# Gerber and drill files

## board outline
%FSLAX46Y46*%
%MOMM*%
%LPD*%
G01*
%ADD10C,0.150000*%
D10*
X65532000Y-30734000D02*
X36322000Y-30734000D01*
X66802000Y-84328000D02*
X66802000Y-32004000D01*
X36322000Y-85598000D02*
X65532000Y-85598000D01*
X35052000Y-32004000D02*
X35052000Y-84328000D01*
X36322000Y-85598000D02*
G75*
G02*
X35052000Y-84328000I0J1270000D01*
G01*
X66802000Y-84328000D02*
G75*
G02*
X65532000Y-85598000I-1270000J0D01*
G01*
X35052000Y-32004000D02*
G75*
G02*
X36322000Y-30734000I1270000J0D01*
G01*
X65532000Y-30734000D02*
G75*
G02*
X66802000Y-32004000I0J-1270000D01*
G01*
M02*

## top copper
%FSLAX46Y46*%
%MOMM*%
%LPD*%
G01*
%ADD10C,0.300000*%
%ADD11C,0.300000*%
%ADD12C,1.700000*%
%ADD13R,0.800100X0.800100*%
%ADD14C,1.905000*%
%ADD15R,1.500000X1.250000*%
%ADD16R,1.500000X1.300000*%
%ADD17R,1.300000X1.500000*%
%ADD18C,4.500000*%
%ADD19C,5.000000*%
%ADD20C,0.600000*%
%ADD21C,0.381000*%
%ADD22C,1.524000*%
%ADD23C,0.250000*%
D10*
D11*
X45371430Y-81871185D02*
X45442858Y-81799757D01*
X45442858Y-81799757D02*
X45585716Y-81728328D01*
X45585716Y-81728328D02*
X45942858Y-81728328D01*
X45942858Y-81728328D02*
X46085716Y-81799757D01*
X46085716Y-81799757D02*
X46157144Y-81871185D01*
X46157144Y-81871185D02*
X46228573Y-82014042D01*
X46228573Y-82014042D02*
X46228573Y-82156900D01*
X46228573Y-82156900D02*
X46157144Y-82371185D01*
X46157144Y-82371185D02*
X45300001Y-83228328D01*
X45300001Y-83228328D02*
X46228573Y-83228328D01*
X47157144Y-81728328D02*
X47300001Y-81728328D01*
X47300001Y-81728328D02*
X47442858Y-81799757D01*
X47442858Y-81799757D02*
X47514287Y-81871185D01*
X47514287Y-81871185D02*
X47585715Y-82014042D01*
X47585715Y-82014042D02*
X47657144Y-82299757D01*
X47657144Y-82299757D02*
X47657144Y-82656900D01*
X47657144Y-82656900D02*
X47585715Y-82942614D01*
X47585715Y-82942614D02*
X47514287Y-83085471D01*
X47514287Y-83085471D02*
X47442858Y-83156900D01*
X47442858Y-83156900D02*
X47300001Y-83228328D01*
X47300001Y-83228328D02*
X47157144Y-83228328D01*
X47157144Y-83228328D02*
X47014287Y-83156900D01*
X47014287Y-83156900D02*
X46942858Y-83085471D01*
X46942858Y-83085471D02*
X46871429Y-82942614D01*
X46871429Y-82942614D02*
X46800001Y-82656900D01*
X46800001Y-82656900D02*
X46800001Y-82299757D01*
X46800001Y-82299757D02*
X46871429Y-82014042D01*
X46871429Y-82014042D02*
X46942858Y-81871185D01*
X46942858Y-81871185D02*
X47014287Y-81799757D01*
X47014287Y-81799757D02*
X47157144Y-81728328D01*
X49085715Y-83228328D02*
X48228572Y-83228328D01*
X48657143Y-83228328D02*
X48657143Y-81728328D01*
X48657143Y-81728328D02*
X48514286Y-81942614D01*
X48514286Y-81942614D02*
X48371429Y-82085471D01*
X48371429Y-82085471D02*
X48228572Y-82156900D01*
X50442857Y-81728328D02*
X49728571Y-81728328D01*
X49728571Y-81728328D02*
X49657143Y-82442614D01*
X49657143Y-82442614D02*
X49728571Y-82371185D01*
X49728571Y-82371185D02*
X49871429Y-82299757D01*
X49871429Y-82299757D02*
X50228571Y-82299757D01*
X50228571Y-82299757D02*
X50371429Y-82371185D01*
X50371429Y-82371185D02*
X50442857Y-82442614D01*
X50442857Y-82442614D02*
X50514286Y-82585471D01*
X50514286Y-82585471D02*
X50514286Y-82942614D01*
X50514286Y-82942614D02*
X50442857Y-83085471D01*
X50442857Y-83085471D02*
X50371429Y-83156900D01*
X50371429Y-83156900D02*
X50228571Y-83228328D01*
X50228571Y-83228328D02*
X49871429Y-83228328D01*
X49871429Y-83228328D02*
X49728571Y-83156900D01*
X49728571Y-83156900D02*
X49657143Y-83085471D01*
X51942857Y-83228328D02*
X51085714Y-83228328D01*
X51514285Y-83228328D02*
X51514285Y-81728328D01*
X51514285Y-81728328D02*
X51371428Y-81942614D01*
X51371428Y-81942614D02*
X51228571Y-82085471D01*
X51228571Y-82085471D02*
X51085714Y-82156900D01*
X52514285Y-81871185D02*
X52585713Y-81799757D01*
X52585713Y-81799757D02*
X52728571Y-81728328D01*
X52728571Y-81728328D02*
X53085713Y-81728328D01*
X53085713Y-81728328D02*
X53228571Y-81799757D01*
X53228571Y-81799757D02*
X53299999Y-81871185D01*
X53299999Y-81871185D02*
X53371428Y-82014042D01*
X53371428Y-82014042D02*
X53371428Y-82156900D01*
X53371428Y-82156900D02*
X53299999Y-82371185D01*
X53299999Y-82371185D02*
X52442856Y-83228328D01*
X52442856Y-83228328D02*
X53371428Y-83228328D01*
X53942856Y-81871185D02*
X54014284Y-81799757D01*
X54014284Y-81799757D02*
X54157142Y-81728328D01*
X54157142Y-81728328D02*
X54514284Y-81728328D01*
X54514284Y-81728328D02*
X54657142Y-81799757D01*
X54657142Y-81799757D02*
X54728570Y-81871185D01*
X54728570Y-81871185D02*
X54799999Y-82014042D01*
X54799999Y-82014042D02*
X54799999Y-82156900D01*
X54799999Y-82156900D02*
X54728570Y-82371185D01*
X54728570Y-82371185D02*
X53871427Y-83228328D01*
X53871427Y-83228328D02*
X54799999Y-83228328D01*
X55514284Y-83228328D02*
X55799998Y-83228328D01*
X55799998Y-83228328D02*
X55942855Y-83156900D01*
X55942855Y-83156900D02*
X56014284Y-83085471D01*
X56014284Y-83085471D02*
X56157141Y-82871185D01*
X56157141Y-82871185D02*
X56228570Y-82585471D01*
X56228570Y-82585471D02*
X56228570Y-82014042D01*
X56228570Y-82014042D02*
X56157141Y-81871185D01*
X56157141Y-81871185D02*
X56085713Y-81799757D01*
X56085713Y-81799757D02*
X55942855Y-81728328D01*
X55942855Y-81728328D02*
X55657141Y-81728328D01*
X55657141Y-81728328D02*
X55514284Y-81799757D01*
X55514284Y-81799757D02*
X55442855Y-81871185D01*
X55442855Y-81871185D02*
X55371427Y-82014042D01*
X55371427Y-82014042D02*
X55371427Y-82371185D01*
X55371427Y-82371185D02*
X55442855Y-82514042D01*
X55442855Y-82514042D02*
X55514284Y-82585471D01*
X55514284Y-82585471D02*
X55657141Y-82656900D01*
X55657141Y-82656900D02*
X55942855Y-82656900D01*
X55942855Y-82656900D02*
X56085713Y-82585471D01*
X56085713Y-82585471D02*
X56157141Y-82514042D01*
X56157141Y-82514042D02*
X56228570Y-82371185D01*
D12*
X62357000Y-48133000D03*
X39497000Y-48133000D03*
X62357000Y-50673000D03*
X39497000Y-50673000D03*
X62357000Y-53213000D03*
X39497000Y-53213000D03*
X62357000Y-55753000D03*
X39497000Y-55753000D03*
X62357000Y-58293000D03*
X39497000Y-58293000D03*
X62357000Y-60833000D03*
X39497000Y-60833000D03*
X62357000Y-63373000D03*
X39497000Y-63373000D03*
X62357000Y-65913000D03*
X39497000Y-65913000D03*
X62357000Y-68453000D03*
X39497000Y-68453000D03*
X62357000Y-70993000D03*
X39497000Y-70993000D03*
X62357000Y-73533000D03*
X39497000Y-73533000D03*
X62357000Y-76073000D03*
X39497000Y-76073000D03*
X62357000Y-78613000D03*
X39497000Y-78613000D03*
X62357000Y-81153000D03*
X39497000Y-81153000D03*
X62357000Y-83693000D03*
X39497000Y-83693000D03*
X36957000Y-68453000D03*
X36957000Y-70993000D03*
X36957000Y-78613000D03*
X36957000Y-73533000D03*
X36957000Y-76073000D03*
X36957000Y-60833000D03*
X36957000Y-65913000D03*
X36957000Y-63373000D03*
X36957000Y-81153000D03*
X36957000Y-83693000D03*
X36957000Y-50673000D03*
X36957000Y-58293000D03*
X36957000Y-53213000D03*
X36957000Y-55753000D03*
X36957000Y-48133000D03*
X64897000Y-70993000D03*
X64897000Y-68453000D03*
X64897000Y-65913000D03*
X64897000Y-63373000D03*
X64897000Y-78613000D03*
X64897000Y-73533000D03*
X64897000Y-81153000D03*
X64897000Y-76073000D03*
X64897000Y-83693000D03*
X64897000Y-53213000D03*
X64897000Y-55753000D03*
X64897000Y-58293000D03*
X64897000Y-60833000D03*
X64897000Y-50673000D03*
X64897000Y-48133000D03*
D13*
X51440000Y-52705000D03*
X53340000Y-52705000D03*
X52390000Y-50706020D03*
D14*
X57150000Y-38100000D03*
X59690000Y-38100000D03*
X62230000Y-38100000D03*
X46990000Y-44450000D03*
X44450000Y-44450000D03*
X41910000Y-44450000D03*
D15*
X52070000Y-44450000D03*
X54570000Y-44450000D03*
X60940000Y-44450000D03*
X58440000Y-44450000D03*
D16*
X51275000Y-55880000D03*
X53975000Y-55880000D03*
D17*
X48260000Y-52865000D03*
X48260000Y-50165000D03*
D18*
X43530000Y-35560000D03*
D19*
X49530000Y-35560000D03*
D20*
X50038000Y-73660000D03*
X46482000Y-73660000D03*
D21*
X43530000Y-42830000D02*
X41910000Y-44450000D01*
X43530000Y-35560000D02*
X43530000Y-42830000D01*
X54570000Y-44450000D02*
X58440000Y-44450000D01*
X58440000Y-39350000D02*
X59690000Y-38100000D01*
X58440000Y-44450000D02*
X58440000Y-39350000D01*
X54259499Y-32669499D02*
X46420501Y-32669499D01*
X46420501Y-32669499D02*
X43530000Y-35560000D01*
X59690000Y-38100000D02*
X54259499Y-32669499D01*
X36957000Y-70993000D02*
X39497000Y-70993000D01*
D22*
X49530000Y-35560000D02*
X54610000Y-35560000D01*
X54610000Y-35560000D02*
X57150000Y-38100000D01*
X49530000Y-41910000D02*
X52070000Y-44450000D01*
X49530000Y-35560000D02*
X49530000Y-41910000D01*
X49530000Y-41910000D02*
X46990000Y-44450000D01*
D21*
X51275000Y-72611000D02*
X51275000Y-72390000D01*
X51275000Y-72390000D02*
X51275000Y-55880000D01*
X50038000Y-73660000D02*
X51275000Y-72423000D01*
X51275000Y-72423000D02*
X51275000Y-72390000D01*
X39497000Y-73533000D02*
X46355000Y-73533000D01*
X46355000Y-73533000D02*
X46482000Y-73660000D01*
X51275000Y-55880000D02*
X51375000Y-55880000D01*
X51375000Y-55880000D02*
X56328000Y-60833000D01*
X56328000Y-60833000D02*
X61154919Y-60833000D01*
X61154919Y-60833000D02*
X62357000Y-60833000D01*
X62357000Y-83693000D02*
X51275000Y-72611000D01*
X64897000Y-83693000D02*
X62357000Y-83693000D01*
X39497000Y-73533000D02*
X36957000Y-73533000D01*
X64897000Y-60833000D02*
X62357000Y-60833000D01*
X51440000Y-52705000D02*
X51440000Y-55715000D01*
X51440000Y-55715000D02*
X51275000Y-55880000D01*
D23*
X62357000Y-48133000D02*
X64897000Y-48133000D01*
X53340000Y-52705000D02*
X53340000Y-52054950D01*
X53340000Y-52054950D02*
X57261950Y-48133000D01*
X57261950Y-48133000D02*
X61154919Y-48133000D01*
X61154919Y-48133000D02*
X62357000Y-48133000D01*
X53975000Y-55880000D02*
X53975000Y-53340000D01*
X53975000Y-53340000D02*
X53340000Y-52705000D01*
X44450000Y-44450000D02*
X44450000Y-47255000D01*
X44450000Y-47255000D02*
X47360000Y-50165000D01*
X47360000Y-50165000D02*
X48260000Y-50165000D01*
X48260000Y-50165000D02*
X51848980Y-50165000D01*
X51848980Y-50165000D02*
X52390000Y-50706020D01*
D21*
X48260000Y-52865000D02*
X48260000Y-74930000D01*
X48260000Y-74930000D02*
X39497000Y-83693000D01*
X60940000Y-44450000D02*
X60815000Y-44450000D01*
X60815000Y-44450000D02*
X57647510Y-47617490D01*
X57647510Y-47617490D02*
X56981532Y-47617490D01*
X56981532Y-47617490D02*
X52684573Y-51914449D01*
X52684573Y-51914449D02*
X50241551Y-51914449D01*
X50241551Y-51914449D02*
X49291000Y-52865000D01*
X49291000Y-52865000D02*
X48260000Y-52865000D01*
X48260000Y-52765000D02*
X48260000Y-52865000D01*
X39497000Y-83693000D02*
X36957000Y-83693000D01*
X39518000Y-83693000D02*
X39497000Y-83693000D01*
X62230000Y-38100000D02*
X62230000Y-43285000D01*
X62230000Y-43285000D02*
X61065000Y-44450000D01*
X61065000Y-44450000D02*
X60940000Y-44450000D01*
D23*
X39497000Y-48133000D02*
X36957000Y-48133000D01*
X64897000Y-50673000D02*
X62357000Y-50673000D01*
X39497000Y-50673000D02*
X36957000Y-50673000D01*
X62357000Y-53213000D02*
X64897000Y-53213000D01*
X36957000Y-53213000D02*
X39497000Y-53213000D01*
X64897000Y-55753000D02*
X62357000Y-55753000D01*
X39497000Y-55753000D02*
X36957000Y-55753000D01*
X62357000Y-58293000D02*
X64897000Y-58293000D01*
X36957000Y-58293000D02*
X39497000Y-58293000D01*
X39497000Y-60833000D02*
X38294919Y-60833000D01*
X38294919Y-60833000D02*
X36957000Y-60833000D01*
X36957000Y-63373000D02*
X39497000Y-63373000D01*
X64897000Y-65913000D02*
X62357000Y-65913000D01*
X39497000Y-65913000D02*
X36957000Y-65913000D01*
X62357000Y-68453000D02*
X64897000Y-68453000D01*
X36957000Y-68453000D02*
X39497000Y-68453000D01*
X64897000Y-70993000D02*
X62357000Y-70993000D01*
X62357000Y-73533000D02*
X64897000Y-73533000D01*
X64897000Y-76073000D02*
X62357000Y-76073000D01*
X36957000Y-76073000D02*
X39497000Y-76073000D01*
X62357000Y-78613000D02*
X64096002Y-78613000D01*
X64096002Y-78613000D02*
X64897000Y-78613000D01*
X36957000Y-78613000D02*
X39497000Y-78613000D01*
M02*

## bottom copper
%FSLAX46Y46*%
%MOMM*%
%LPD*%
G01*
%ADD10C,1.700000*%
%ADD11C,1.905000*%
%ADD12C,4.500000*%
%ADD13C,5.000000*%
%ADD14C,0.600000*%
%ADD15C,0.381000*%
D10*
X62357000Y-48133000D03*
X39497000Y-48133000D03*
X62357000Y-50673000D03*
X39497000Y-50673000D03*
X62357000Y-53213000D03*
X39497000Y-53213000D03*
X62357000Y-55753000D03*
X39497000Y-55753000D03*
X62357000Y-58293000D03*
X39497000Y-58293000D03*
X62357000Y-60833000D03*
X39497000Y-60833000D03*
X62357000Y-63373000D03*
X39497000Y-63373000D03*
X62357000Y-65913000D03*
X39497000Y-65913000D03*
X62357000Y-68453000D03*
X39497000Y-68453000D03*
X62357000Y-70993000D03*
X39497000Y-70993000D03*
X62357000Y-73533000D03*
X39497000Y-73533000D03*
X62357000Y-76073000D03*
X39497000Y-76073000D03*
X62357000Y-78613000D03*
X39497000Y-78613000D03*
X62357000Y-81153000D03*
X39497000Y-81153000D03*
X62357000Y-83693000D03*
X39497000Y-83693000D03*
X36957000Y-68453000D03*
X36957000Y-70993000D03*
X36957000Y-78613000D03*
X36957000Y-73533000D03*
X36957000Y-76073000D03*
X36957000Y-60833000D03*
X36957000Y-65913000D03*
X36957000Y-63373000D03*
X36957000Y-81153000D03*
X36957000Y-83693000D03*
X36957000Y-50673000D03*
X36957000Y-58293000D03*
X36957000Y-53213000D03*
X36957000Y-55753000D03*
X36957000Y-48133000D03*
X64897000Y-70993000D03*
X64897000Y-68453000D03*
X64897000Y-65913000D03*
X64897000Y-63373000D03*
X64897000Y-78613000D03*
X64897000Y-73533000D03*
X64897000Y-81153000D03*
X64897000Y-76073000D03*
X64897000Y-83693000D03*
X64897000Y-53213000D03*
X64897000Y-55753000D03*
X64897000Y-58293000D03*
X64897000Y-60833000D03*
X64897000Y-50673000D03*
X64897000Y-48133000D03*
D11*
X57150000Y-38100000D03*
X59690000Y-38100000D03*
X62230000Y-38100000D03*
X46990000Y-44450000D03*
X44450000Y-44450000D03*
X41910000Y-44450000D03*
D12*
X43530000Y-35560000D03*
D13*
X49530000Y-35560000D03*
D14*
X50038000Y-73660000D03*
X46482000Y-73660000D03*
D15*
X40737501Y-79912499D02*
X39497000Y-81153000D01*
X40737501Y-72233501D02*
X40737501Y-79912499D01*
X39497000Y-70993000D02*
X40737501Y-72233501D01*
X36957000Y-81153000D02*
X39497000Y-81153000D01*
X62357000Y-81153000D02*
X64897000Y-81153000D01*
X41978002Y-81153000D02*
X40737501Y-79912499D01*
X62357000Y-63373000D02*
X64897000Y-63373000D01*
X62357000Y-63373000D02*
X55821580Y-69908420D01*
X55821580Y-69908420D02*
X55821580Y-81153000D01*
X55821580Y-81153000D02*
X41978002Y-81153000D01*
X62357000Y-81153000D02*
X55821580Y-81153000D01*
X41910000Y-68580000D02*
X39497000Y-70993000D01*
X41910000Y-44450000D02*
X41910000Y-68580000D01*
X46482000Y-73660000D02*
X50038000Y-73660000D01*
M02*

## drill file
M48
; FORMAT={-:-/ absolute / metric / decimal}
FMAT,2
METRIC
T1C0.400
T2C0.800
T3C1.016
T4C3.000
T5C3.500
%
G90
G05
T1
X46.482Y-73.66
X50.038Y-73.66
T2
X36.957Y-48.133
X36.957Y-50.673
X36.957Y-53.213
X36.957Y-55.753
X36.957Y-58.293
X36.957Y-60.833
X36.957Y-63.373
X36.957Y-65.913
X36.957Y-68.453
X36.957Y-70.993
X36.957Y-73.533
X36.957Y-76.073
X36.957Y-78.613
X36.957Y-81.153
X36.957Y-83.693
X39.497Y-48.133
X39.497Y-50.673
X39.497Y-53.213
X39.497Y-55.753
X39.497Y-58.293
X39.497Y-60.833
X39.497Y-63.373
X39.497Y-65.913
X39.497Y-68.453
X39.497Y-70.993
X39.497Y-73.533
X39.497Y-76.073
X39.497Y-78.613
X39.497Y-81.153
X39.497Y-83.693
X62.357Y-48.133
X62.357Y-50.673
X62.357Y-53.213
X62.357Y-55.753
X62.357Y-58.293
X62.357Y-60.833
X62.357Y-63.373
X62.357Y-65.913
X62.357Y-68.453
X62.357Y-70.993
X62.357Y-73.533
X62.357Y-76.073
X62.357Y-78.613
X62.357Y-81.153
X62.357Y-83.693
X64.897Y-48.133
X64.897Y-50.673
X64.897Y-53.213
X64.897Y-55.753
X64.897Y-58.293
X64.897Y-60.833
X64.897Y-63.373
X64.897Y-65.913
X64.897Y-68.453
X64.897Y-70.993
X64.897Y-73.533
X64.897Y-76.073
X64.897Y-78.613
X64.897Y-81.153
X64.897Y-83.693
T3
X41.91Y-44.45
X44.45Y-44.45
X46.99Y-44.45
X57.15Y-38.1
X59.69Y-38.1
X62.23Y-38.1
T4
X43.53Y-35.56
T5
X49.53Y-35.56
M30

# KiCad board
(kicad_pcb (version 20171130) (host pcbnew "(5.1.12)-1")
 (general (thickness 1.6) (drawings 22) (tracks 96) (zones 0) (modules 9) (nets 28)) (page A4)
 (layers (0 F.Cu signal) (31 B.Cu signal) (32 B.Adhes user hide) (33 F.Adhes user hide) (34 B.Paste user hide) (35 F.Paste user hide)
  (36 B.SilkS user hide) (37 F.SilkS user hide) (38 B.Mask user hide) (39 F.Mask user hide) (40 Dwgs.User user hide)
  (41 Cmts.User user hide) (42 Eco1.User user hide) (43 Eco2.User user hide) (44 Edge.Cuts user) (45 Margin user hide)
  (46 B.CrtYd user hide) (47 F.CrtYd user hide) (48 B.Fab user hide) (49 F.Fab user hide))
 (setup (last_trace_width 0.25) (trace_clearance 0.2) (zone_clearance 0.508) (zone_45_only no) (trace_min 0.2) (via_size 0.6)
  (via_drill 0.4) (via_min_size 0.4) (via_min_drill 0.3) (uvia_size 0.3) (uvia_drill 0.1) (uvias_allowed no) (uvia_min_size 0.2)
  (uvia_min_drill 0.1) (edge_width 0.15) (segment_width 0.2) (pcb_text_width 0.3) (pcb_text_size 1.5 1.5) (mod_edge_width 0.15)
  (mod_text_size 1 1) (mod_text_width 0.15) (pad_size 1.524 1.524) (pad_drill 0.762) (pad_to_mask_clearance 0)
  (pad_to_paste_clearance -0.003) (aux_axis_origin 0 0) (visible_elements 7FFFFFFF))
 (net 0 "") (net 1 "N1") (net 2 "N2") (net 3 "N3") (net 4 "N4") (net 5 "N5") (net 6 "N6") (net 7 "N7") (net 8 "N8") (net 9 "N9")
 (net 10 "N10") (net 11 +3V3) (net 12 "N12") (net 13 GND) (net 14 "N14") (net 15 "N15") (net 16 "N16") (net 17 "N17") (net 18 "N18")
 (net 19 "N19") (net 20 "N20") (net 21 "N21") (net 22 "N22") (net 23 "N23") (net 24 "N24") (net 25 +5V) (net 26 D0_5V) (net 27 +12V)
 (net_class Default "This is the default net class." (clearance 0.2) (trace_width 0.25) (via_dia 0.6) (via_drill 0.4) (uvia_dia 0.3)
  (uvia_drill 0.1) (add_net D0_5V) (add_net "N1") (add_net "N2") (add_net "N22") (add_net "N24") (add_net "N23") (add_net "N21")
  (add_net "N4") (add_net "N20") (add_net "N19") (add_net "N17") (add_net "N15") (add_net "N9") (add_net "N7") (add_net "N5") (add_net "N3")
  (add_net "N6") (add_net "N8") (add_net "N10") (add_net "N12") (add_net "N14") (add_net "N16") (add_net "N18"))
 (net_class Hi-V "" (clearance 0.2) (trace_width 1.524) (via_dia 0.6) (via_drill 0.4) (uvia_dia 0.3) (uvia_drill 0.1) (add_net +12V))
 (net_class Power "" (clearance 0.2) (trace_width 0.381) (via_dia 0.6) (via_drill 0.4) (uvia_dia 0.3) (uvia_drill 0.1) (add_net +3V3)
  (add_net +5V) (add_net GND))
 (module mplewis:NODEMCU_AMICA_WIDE (layer F.Cu) (at 50.8 66.04)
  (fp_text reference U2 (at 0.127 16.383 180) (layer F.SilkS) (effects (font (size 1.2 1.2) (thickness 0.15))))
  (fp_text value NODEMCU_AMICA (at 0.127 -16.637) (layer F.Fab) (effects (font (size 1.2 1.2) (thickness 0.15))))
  (pad 30 thru_hole circle (at 11.557 -17.907 270) (size 1.7 1.7) (drill 0.8) (layers *.Cu *.Mask F.SilkS) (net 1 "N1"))
  (pad 1 thru_hole circle (at -11.303 -17.907 270) (size 1.7 1.7) (drill 0.8) (layers *.Cu *.Mask F.SilkS) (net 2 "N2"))
  (pad 29 thru_hole circle (at 11.557 -15.367 270) (size 1.7 1.7) (drill 0.8) (layers *.Cu *.Mask F.SilkS) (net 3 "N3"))
  (pad 2 thru_hole circle (at -11.303 -15.367 270) (size 1.7 1.7) (drill 0.8) (layers *.Cu *.Mask F.SilkS) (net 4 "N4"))
  (pad 28 thru_hole circle (at 11.557 -12.827 270) (size 1.7 1.7) (drill 0.8) (layers *.Cu *.Mask F.SilkS) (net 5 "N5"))
  (pad 3 thru_hole circle (at -11.303 -12.827 270) (size 1.7 1.7) (drill 0.8) (layers *.Cu *.Mask F.SilkS) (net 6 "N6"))
  (pad 27 thru_hole circle (at 11.557 -10.287 270) (size 1.7 1.7) (drill 0.8) (layers *.Cu *.Mask F.SilkS) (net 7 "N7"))
  (pad 4 thru_hole circle (at -11.303 -10.287 270) (size 1.7 1.7) (drill 0.8) (layers *.Cu *.Mask F.SilkS) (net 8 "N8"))
  (pad 26 thru_hole circle (at 11.557 -7.747 270) (size 1.7 1.7) (drill 0.8) (layers *.Cu *.Mask F.SilkS) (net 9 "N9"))
  (pad 5 thru_hole circle (at -11.303 -7.747 270) (size 1.7 1.7) (drill 0.8) (layers *.Cu *.Mask F.SilkS) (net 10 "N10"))
  (pad 25 thru_hole circle (at 11.557 -5.207 270) (size 1.7 1.7) (drill 0.8) (layers *.Cu *.Mask F.SilkS) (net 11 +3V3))
  (pad 6 thru_hole circle (at -11.303 -5.207 270) (size 1.7 1.7) (drill 0.8) (layers *.Cu *.Mask F.SilkS) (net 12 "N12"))
  (pad 24 thru_hole circle (at 11.557 -2.667 270) (size 1.7 1.7) (drill 0.8) (layers *.Cu *.Mask F.SilkS) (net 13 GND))
  (pad 7 thru_hole circle (at -11.303 -2.667 270) (size 1.7 1.7) (drill 0.8) (layers *.Cu *.Mask F.SilkS) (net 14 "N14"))
  (pad 23 thru_hole circle (at 11.557 -0.127 270) (size 1.7 1.7) (drill 0.8) (layers *.Cu *.Mask F.SilkS) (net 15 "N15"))
  (pad 8 thru_hole circle (at -11.303 -0.127 270) (size 1.7 1.7) (drill 0.8) (layers *.Cu *.Mask F.SilkS) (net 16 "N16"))
  (pad 22 thru_hole circle (at 11.557 2.413 270) (size 1.7 1.7) (drill 0.8) (layers *.Cu *.Mask F.SilkS) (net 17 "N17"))
  (pad 9 thru_hole circle (at -11.303 2.413 270) (size 1.7 1.7) (drill 0.8) (layers *.Cu *.Mask F.SilkS) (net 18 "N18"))
  (pad 21 thru_hole circle (at 11.557 4.953 270) (size 1.7 1.7) (drill 0.8) (layers *.Cu *.Mask F.SilkS) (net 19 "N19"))
  (pad 10 thru_hole circle (at -11.303 4.953 270) (size 1.7 1.7) (drill 0.8) (layers *.Cu *.Mask F.SilkS) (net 13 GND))
  (pad 20 thru_hole circle (at 11.557 7.493 270) (size 1.7 1.7) (drill 0.8) (layers *.Cu *.Mask F.SilkS) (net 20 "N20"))
  (pad 11 thru_hole circle (at -11.303 7.493 270) (size 1.7 1.7) (drill 0.8) (layers *.Cu *.Mask F.SilkS) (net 11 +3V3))
  (pad 19 thru_hole circle (at 11.557 10.033 270) (size 1.7 1.7) (drill 0.8) (layers *.Cu *.Mask F.SilkS) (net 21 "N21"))
  (pad 12 thru_hole circle (at -11.303 10.033 270) (size 1.7 1.7) (drill 0.8) (layers *.Cu *.Mask F.SilkS) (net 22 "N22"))
  (pad 18 thru_hole circle (at 11.557 12.573 270) (size 1.7 1.7) (drill 0.8) (layers *.Cu *.Mask F.SilkS) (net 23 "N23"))
  (pad 13 thru_hole circle (at -11.303 12.573 270) (size 1.7 1.7) (drill 0.8) (layers *.Cu *.Mask F.SilkS) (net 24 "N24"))
  (pad 17 thru_hole circle (at 11.557 15.113 270) (size 1.7 1.7) (drill 0.8) (layers *.Cu *.Mask F.SilkS) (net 13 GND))
  (pad 14 thru_hole circle (at -11.303 15.113 270) (size 1.7 1.7) (drill 0.8) (layers *.Cu *.Mask F.SilkS) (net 13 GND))
  (pad 16 thru_hole circle (at 11.557 17.653 270) (size 1.7 1.7) (drill 0.8) (layers *.Cu *.Mask F.SilkS) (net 11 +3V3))
  (pad 15 thru_hole circle (at -11.303 17.653 270) (size 1.7 1.7) (drill 0.8) (layers *.Cu *.Mask F.SilkS) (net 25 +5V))
  (pad 9 thru_hole circle (at -13.843 2.413 270) (size 1.7 1.7) (drill 0.8) (layers *.Cu *.Mask F.SilkS) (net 18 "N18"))
  (pad 10 thru_hole circle (at -13.843 4.953 270) (size 1.7 1.7) (drill 0.8) (layers *.Cu *.Mask F.SilkS) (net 13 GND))
  (pad 13 thru_hole circle (at -13.843 12.573 270) (size 1.7 1.7) (drill 0.8) (layers *.Cu *.Mask F.SilkS) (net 24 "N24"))
  (pad 11 thru_hole circle (at -13.843 7.493 270) (size 1.7 1.7) (drill 0.8) (layers *.Cu *.Mask F.SilkS) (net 11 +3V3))
  (pad 12 thru_hole circle (at -13.843 10.033 270) (size 1.7 1.7) (drill 0.8) (layers *.Cu *.Mask F.SilkS) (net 22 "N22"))
  (pad 6 thru_hole circle (at -13.843 -5.207 270) (size 1.7 1.7) (drill 0.8) (layers *.Cu *.Mask F.SilkS) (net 12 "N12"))
  (pad 8 thru_hole circle (at -13.843 -0.127 270) (size 1.7 1.7) (drill 0.8) (layers *.Cu *.Mask F.SilkS) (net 16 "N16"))
  (pad 7 thru_hole circle (at -13.843 -2.667 270) (size 1.7 1.7) (drill 0.8) (layers *.Cu *.Mask F.SilkS) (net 14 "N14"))
  (pad 14 thru_hole circle (at -13.843 15.113 270) (size 1.7 1.7) (drill 0.8) (layers *.Cu *.Mask F.SilkS) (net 13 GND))
  (pad 15 thru_hole circle (at -13.843 17.653 270) (size 1.7 1.7) (drill 0.8) (layers *.Cu *.Mask F.SilkS) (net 25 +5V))
  (pad 2 thru_hole circle (at -13.843 -15.367 270) (size 1.7 1.7) (drill 0.8) (layers *.Cu *.Mask F.SilkS) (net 4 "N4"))
  (pad 5 thru_hole circle (at -13.843 -7.747 270) (size 1.7 1.7) (drill 0.8) (layers *.Cu *.Mask F.SilkS) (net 10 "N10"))
  (pad 3 thru_hole circle (at -13.843 -12.827 270) (size 1.7 1.7) (drill 0.8) (layers *.Cu *.Mask F.SilkS) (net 6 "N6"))
  (pad 4 thru_hole circle (at -13.843 -10.287 270) (size 1.7 1.7) (drill 0.8) (layers *.Cu *.Mask F.SilkS) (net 8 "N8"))
  (pad 1 thru_hole circle (at -13.843 -17.907 270) (size 1.7 1.7) (drill 0.8) (layers *.Cu *.Mask F.SilkS) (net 2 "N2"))
  (pad 21 thru_hole circle (at 14.097 4.953 270) (size 1.7 1.7) (drill 0.8) (layers *.Cu *.Mask F.SilkS) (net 19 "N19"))
  (pad 22 thru_hole circle (at 14.097 2.413 270) (size 1.7 1.7) (drill 0.8) (layers *.Cu *.Mask F.SilkS) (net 17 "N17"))
  (pad 23 thru_hole circle (at 14.097 -0.127 270) (size 1.7 1.7) (drill 0.8) (layers *.Cu *.Mask F.SilkS) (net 15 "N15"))
  (pad 24 thru_hole circle (at 14.097 -2.667 270) (size 1.7 1.7) (drill 0.8) (layers *.Cu *.Mask F.SilkS) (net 13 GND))
  (pad 18 thru_hole circle (at 14.097 12.573 270) (size 1.7 1.7) (drill 0.8) (layers *.Cu *.Mask F.SilkS) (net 23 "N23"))
  (pad 20 thru_hole circle (at 14.097 7.493 270) (size 1.7 1.7) (drill 0.8) (layers *.Cu *.Mask F.SilkS) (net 20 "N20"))
  (pad 17 thru_hole circle (at 14.097 15.113 270) (size 1.7 1.7) (drill 0.8) (layers *.Cu *.Mask F.SilkS) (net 13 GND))
  (pad 19 thru_hole circle (at 14.097 10.033 270) (size 1.7 1.7) (drill 0.8) (layers *.Cu *.Mask F.SilkS) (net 21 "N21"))
  (pad 16 thru_hole circle (at 14.097 17.653 270) (size 1.7 1.7) (drill 0.8) (layers *.Cu *.Mask F.SilkS) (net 11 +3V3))
  (pad 28 thru_hole circle (at 14.097 -12.827 270) (size 1.7 1.7) (drill 0.8) (layers *.Cu *.Mask F.SilkS) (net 5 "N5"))
  (pad 27 thru_hole circle (at 14.097 -10.287 270) (size 1.7 1.7) (drill 0.8) (layers *.Cu *.Mask F.SilkS) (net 7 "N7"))
  (pad 26 thru_hole circle (at 14.097 -7.747 270) (size 1.7 1.7) (drill 0.8) (layers *.Cu *.Mask F.SilkS) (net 9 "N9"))
  (pad 25 thru_hole circle (at 14.097 -5.207 270) (size 1.7 1.7) (drill 0.8) (layers *.Cu *.Mask F.SilkS) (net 11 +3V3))
  (pad 29 thru_hole circle (at 14.097 -15.367 270) (size 1.7 1.7) (drill 0.8) (layers *.Cu *.Mask F.SilkS) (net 3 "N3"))
  (pad 30 thru_hole circle (at 14.097 -17.907 270) (size 1.7 1.7) (drill 0.8) (layers *.Cu *.Mask F.SilkS) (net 1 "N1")))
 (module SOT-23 (layer F.Cu) (at 52.39 51.70424)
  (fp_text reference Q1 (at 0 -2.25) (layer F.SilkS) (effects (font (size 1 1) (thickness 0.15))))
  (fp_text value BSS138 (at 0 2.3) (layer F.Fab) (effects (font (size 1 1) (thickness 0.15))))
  (pad 1 smd rect (at -0.95 1.00076) (size 0.8001 0.8001) (layers F.Cu F.Paste F.Mask) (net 11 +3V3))
  (pad 2 smd rect (at 0.95 1.00076) (size 0.8001 0.8001) (layers F.Cu F.Paste F.Mask) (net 1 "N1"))
  (pad 3 smd rect (at 0 -0.99822) (size 0.8001 0.8001) (layers F.Cu F.Paste F.Mask) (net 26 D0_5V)))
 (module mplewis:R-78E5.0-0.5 (layer F.Cu) (at 59.69 40.132)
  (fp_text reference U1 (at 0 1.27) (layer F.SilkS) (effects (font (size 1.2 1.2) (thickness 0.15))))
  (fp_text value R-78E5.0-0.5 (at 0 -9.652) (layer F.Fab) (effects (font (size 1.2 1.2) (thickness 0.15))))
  (pad 1 thru_hole circle (at -2.54 -2.032) (size 1.905 1.905) (drill 1.016) (layers *.Cu *.Mask F.SilkS) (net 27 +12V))
  (pad 2 thru_hole circle (at 0 -2.032) (size 1.905 1.905) (drill 1.016) (layers *.Cu *.Mask F.SilkS) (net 13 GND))
  (pad 3 thru_hole circle (at 2.54 -2.032) (size 1.905 1.905) (drill 1.016) (layers *.Cu *.Mask F.SilkS) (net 25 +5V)))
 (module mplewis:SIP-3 (layer F.Cu) (at 44.45 44.45 180)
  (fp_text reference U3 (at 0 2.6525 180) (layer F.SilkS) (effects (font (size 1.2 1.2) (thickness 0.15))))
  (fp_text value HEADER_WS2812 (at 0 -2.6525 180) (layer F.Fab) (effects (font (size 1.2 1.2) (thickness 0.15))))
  (pad 1 thru_hole circle (at -2.54 0 180) (size 1.905 1.905) (drill 1.016) (layers *.Cu *.Mask F.SilkS) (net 27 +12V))
  (pad 2 thru_hole circle (at 0 0 180) (size 1.905 1.905) (drill 1.016) (layers *.Cu *.Mask F.SilkS) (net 26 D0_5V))
  (pad 3 thru_hole circle (at 2.54 0 180) (size 1.905 1.905) (drill 1.016) (layers *.Cu *.Mask F.SilkS) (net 13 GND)))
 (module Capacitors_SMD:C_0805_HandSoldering (layer F.Cu) (at 53.32 44.45)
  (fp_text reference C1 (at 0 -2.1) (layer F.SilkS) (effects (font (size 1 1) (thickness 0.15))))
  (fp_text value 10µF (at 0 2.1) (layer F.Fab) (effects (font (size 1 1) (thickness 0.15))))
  (pad 1 smd rect (at -1.25 0) (size 1.5 1.25) (layers F.Cu F.Paste F.Mask) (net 27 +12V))
  (pad 2 smd rect (at 1.25 0) (size 1.5 1.25) (layers F.Cu F.Paste F.Mask) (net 13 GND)))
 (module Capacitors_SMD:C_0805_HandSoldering (layer F.Cu) (at 59.69 44.45 180)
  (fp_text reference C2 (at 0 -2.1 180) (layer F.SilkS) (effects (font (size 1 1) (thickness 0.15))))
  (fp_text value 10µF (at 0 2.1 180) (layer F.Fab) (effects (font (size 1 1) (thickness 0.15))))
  (pad 1 smd rect (at -1.25 0 180) (size 1.5 1.25) (layers F.Cu F.Paste F.Mask) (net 25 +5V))
  (pad 2 smd rect (at 1.25 0 180) (size 1.5 1.25) (layers F.Cu F.Paste F.Mask) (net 13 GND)))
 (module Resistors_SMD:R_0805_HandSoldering (layer F.Cu) (at 52.625 55.88)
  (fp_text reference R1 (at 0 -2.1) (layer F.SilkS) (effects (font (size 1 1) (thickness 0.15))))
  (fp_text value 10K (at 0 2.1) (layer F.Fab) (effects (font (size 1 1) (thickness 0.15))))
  (pad 1 smd rect (at -1.35 0) (size 1.5 1.3) (layers F.Cu F.Paste F.Mask) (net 11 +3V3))
  (pad 2 smd rect (at 1.35 0) (size 1.5 1.3) (layers F.Cu F.Paste F.Mask) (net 1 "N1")))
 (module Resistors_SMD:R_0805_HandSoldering (layer F.Cu) (at 48.26 51.515 90)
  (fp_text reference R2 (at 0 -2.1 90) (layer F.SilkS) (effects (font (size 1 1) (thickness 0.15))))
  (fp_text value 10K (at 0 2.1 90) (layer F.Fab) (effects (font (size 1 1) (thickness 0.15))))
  (pad 1 smd rect (at -1.35 0 90) (size 1.5 1.3) (layers F.Cu F.Paste F.Mask) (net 25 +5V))
  (pad 2 smd rect (at 1.35 0 90) (size 1.5 1.3) (layers F.Cu F.Paste F.Mask) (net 26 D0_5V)))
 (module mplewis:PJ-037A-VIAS (layer F.Cu) (at 43.53 35.56)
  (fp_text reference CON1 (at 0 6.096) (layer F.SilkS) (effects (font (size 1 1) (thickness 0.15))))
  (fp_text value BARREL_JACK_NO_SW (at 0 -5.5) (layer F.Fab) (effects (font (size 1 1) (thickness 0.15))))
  (pad 2 thru_hole circle (at 0 0) (size 4.5 4.5) (drill 3) (layers *.Cu *.Mask F.SilkS) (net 13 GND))
  (pad 1 thru_hole circle (at 6 0) (size 5 5) (drill 3.5) (layers *.Cu *.Mask F.SilkS) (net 27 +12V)))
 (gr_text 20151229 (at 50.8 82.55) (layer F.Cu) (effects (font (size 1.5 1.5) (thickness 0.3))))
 (gr_line (start 65.532 30.734) (end 36.322 30.734) (layer Edge.Cuts) (width 0.15))
 (gr_line (start 66.802 84.328) (end 66.802 32.004) (layer Edge.Cuts) (width 0.15))
 (gr_line (start 36.322 85.598) (end 65.532 85.598) (layer Edge.Cuts) (width 0.15))
 (gr_line (start 35.052 32.004) (end 35.052 84.328) (layer Edge.Cuts) (width 0.15))
 (gr_arc (start 36.322 84.328) (end 36.322 85.598) (angle 90) (layer Edge.Cuts) (width 0.15))
 (gr_arc (start 65.532 84.328) (end 66.802 84.328) (angle 90) (layer Edge.Cuts) (width 0.15))
 (gr_arc (start 36.322 32.004) (end 35.052 32.004) (angle 90) (layer Edge.Cuts) (width 0.15))
 (gr_arc (start 65.532 32.004) (end 65.532 30.734) (angle 90) (layer Edge.Cuts) (width 0.15))
 (segment (start 43.53 42.83) (end 41.91 44.45) (width 0.381) (layer F.Cu) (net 13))
 (segment (start 43.53 35.56) (end 43.53 42.83) (width 0.381) (layer F.Cu) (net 13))
 (segment (start 54.57 44.45) (end 58.44 44.45) (width 0.381) (layer F.Cu) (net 13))
 (segment (start 58.44 39.35) (end 59.69 38.1) (width 0.381) (layer F.Cu) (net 13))
 (segment (start 58.44 44.45) (end 58.44 39.35) (width 0.381) (layer F.Cu) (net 13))
 (segment (start 54.259499 32.669499) (end 46.420501 32.669499) (width 0.381) (layer F.Cu) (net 13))
 (segment (start 46.420501 32.669499) (end 43.53 35.56) (width 0.381) (layer F.Cu) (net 13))
 (segment (start 59.69 38.1) (end 54.259499 32.669499) (width 0.381) (layer F.Cu) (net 13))
 (segment (start 36.957 70.993) (end 39.497 70.993) (width 0.381) (layer F.Cu) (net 13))
 (segment (start 40.737501 79.912499) (end 39.497 81.153) (width 0.381) (layer B.Cu) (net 13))
 (segment (start 40.737501 72.233501) (end 40.737501 79.912499) (width 0.381) (layer B.Cu) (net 13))
 (segment (start 39.497 70.993) (end 40.737501 72.233501) (width 0.381) (layer B.Cu) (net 13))
 (segment (start 36.957 81.153) (end 39.497 81.153) (width 0.381) (layer B.Cu) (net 13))
 (segment (start 62.357 81.153) (end 64.897 81.153) (width 0.381) (layer B.Cu) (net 13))
 (segment (start 41.978002 81.153) (end 40.737501 79.912499) (width 0.381) (layer B.Cu) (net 13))
 (segment (start 62.357 63.373) (end 64.897 63.373) (width 0.381) (layer B.Cu) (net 13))
 (segment (start 62.357 63.373) (end 55.82158 69.90842) (width 0.381) (layer B.Cu) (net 13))
 (segment (start 55.82158 69.90842) (end 55.82158 81.153) (width 0.381) (layer B.Cu) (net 13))
 (segment (start 55.82158 81.153) (end 41.978002 81.153) (width 0.381) (layer B.Cu) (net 13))
 (segment (start 62.357 81.153) (end 55.82158 81.153) (width 0.381) (layer B.Cu) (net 13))
 (segment (start 41.91 68.58) (end 39.497 70.993) (width 0.381) (layer B.Cu) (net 13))
 (segment (start 41.91 44.45) (end 41.91 68.58) (width 0.381) (layer B.Cu) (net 13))
 (segment (start 49.53 35.56) (end 54.61 35.56) (width 1.524) (layer F.Cu) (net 27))
 (segment (start 54.61 35.56) (end 57.15 38.1) (width 1.524) (layer F.Cu) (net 27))
 (segment (start 49.53 41.91) (end 52.07 44.45) (width 1.524) (layer F.Cu) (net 27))
 (segment (start 49.53 35.56) (end 49.53 41.91) (width 1.524) (layer F.Cu) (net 27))
 (segment (start 49.53 41.91) (end 46.99 44.45) (width 1.524) (layer F.Cu) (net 27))
 (segment (start 51.275 72.611) (end 51.275 72.39) (width 0.381) (layer F.Cu) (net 11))
 (segment (start 51.275 72.39) (end 51.275 55.88) (width 0.381) (layer F.Cu) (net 11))
 (segment (start 50.038 73.66) (end 51.275 72.423) (width 0.381) (layer F.Cu) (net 11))
 (segment (start 51.275 72.423) (end 51.275 72.39) (width 0.381) (layer F.Cu) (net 11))
 (segment (start 46.482 73.66) (end 50.038 73.66) (width 0.381) (layer B.Cu) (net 11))
 (segment (start 39.497 73.533) (end 46.355 73.533) (width 0.381) (layer F.Cu) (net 11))
 (segment (start 46.355 73.533) (end 46.482 73.66) (width 0.381) (layer F.Cu) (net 11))
 (segment (start 51.275 55.88) (end 51.375 55.88) (width 0.381) (layer F.Cu) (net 11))
 (segment (start 51.375 55.88) (end 56.328 60.833) (width 0.381) (layer F.Cu) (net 11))
 (segment (start 56.328 60.833) (end 61.154919 60.833) (width 0.381) (layer F.Cu) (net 11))
 (segment (start 61.154919 60.833) (end 62.357 60.833) (width 0.381) (layer F.Cu) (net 11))
 (segment (start 62.357 83.693) (end 51.275 72.611) (width 0.381) (layer F.Cu) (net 11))
 (segment (start 64.897 83.693) (end 62.357 83.693) (width 0.381) (layer F.Cu) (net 11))
 (segment (start 39.497 73.533) (end 36.957 73.533) (width 0.381) (layer F.Cu) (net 11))
 (segment (start 64.897 60.833) (end 62.357 60.833) (width 0.381) (layer F.Cu) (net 11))
 (segment (start 51.44 52.705) (end 51.44 55.715) (width 0.381) (layer F.Cu) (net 11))
 (segment (start 51.44 55.715) (end 51.275 55.88) (width 0.381) (layer F.Cu) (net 11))
 (via (at 50.038 73.66) (size 0.6) (drill 0.4) (layers F.Cu B.Cu) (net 11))
 (via (at 46.482 73.66) (size 0.6) (drill 0.4) (layers F.Cu B.Cu) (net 11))
 (segment (start 62.357 48.133) (end 64.897 48.133) (width 0.25) (layer F.Cu) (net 1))
 (segment (start 53.34 52.705) (end 53.34 52.05495) (width 0.25) (layer F.Cu) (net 1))
 (segment (start 53.34 52.05495) (end 57.26195 48.133) (width 0.25) (layer F.Cu) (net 1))
 (segment (start 57.26195 48.133) (end 61.154919 48.133) (width 0.25) (layer F.Cu) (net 1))
 (segment (start 61.154919 48.133) (end 62.357 48.133) (width 0.25) (layer F.Cu) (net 1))
 (segment (start 53.975 55.88) (end 53.975 53.34) (width 0.25) (layer F.Cu) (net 1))
 (segment (start 53.975 53.34) (end 53.34 52.705) (width 0.25) (layer F.Cu) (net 1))
 (segment (start 44.45 44.45) (end 44.45 47.255) (width 0.25) (layer F.Cu) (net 26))
 (segment (start 44.45 47.255) (end 47.36 50.165) (width 0.25) (layer F.Cu) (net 26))
 (segment (start 47.36 50.165) (end 48.26 50.165) (width 0.25) (layer F.Cu) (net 26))
 (segment (start 48.26 50.165) (end 51.84898 50.165) (width 0.25) (layer F.Cu) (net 26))
 (segment (start 51.84898 50.165) (end 52.39 50.70602) (width 0.25) (layer F.Cu) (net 26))
 (segment (start 48.26 52.865) (end 48.26 74.93) (width 0.381) (layer F.Cu) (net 25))
 (segment (start 48.26 74.93) (end 39.497 83.693) (width 0.381) (layer F.Cu) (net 25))
 (segment (start 60.94 44.45) (end 60.815 44.45) (width 0.381) (layer F.Cu) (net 25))
 (segment (start 60.815 44.45) (end 57.64751 47.61749) (width 0.381) (layer F.Cu) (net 25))
 (segment (start 57.64751 47.61749) (end 56.981532 47.61749) (width 0.381) (layer F.Cu) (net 25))
 (segment (start 56.981532 47.61749) (end 52.684573 51.914449) (width 0.381) (layer F.Cu) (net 25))
 (segment (start 52.684573 51.914449) (end 50.241551 51.914449) (width 0.381) (layer F.Cu) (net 25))
 (segment (start 50.241551 51.914449) (end 49.291 52.865) (width 0.381) (layer F.Cu) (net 25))
 (segment (start 49.291 52.865) (end 48.26 52.865) (width 0.381) (layer F.Cu) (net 25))
 (segment (start 48.26 52.765) (end 48.26 52.865) (width 0.381) (layer F.Cu) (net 25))
 (segment (start 39.497 83.693) (end 36.957 83.693) (width 0.381) (layer F.Cu) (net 25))
 (segment (start 39.518 83.693) (end 39.497 83.693) (width 0.381) (layer F.Cu) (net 25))
 (segment (start 62.23 38.1) (end 62.23 43.285) (width 0.381) (layer F.Cu) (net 25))
 (segment (start 62.23 43.285) (end 61.065 44.45) (width 0.381) (layer F.Cu) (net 25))
 (segment (start 61.065 44.45) (end 60.94 44.45) (width 0.381) (layer F.Cu) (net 25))
 (segment (start 39.497 48.133) (end 36.957 48.133) (width 0.25) (layer F.Cu) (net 2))
 (segment (start 64.897 50.673) (end 62.357 50.673) (width 0.25) (layer F.Cu) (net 3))
 (segment (start 39.497 50.673) (end 36.957 50.673) (width 0.25) (layer F.Cu) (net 4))
 (segment (start 62.357 53.213) (end 64.897 53.213) (width 0.25) (layer F.Cu) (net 5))
 (segment (start 36.957 53.213) (end 39.497 53.213) (width 0.25) (layer F.Cu) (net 6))
 (segment (start 64.897 55.753) (end 62.357 55.753) (width 0.25) (layer F.Cu) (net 7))
 (segment (start 39.497 55.753) (end 36.957 55.753) (width 0.25) (layer F.Cu) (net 8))
 (segment (start 62.357 58.293) (end 64.897 58.293) (width 0.25) (layer F.Cu) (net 9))
 (segment (start 36.957 58.293) (end 39.497 58.293) (width 0.25) (layer F.Cu) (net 10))
 (segment (start 39.497 60.833) (end 38.294919 60.833) (width 0.25) (layer F.Cu) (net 12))
 (segment (start 38.294919 60.833) (end 36.957 60.833) (width 0.25) (layer F.Cu) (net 12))
 (segment (start 36.957 63.373) (end 39.497 63.373) (width 0.25) (layer F.Cu) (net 14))
 (segment (start 64.897 65.913) (end 62.357 65.913) (width 0.25) (layer F.Cu) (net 15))
 (segment (start 39.497 65.913) (end 36.957 65.913) (width 0.25) (layer F.Cu) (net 16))
 (segment (start 62.357 68.453) (end 64.897 68.453) (width 0.25) (layer F.Cu) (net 17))
 (segment (start 36.957 68.453) (end 39.497 68.453) (width 0.25) (layer F.Cu) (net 18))
 (segment (start 64.897 70.993) (end 62.357 70.993) (width 0.25) (layer F.Cu) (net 19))
 (segment (start 62.357 73.533) (end 64.897 73.533) (width 0.25) (layer F.Cu) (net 20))
 (segment (start 64.897 76.073) (end 62.357 76.073) (width 0.25) (layer F.Cu) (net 21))
 (segment (start 36.957 76.073) (end 39.497 76.073) (width 0.25) (layer F.Cu) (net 22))
 (segment (start 62.357 78.613) (end 64.096002 78.613) (width 0.25) (layer F.Cu) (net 23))
 (segment (start 64.096002 78.613) (end 64.897 78.613) (width 0.25) (layer F.Cu) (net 23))
 (segment (start 36.957 78.613) (end 39.497 78.613) (width 0.25) (layer F.Cu) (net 24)))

